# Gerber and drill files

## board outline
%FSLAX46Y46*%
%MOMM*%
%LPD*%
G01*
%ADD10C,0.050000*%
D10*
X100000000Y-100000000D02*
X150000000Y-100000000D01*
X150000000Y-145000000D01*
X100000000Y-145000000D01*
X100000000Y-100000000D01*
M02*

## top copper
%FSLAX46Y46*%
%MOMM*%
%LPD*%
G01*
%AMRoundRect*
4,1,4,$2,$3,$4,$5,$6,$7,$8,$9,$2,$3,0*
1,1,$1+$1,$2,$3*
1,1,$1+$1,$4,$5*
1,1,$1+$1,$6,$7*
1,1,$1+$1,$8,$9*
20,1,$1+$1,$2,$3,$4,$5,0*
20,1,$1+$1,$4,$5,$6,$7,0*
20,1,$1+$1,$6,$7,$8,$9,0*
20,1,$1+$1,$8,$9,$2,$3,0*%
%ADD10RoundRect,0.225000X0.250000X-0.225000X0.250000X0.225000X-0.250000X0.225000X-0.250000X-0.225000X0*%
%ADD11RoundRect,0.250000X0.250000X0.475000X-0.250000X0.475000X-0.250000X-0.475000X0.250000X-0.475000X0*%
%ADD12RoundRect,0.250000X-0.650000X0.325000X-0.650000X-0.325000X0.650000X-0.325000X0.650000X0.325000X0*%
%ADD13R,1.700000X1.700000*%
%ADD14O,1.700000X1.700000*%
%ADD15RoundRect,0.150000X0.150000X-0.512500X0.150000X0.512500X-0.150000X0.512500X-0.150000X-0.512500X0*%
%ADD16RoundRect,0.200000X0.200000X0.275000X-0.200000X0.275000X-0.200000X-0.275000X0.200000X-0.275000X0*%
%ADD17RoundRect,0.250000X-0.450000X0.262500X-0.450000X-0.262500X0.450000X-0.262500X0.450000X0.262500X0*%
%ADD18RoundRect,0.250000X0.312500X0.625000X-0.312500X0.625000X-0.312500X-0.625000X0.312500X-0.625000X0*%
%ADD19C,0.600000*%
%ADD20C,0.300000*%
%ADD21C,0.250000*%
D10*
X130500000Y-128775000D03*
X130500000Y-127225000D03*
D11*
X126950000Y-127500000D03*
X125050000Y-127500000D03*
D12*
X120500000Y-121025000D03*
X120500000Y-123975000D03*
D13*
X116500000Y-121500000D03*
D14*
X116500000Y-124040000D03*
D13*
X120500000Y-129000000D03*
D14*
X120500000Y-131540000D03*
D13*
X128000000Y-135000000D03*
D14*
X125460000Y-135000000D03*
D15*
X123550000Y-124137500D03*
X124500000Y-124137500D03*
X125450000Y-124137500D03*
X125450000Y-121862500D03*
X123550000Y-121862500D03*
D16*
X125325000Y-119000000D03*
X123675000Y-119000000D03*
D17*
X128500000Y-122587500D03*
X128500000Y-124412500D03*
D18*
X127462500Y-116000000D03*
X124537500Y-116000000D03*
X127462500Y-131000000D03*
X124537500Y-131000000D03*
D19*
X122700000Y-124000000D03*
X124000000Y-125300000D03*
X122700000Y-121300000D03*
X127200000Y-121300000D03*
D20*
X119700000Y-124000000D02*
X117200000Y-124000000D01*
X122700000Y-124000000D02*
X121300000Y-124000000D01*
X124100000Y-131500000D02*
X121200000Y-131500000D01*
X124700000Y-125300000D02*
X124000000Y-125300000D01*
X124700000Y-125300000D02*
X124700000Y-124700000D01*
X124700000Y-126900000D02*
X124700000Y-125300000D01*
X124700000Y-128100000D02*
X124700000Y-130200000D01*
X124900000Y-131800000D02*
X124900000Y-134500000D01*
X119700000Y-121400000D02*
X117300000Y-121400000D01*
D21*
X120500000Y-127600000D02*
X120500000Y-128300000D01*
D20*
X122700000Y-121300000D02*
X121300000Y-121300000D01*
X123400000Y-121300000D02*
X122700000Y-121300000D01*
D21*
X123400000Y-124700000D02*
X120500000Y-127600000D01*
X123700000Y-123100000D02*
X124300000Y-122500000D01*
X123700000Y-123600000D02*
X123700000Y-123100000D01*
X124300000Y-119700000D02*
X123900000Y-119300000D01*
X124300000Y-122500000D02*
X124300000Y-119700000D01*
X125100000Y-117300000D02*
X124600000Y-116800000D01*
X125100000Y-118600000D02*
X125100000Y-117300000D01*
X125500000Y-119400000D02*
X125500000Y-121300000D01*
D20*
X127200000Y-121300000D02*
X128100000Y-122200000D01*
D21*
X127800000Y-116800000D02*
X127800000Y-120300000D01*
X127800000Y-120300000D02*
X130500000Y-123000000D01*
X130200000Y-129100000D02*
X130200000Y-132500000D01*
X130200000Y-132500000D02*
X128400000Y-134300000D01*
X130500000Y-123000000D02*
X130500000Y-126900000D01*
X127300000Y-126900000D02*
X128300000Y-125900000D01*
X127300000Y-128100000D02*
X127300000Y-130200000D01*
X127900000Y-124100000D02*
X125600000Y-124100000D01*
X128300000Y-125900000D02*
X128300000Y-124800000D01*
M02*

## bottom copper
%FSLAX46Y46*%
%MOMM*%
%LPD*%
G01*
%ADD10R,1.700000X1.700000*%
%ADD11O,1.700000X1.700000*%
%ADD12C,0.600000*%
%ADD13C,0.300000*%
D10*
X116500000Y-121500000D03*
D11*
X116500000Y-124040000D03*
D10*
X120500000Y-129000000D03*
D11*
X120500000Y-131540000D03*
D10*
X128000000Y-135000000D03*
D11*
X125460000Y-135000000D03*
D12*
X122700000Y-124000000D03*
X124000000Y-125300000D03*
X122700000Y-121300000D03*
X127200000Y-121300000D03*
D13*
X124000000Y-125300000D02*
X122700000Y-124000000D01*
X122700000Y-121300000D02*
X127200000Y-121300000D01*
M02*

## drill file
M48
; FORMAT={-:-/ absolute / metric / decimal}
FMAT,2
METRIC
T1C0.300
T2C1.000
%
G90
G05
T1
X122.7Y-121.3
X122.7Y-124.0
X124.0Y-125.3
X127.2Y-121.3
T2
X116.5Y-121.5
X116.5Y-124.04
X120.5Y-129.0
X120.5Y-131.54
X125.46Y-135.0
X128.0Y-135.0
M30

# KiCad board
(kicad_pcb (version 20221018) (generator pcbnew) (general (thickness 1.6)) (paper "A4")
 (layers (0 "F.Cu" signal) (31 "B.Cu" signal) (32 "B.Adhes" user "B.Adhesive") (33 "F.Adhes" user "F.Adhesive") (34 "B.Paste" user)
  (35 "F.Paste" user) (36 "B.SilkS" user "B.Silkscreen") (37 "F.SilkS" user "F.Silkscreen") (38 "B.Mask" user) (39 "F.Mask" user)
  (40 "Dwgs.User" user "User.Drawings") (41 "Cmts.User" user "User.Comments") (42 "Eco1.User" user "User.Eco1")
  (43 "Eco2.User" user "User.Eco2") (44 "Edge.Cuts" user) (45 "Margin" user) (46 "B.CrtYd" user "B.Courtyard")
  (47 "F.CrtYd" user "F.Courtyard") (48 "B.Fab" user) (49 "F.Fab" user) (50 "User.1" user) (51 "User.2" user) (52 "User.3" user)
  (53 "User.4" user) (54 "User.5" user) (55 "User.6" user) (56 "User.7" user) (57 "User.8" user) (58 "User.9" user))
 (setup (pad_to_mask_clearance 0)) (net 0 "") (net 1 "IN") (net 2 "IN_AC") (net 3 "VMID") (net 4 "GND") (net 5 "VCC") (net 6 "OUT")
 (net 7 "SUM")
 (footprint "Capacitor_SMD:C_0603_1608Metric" (layer "F.Cu") (at 130.5 128 90)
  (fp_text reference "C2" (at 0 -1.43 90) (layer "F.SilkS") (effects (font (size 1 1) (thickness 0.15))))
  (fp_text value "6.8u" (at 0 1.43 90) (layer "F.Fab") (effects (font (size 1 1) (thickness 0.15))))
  (pad "1" smd roundrect (at -0.775 0 90) (size 0.9 0.95) (layers "F.Cu" "F.Paste" "F.Mask") (roundrect_rratio 0.25) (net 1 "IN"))
  (pad "2" smd roundrect (at 0.775 0 90) (size 0.9 0.95) (layers "F.Cu" "F.Paste" "F.Mask") (roundrect_rratio 0.25) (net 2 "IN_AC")))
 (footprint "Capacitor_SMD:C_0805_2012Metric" (layer "F.Cu") (at 126 127.5 180)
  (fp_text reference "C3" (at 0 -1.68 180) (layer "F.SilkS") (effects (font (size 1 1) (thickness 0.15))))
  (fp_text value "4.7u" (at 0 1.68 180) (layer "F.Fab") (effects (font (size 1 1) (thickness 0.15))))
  (pad "1" smd roundrect (at -0.95 0 180) (size 1 1.45) (layers "F.Cu" "F.Paste" "F.Mask") (roundrect_rratio 0.25) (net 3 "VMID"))
  (pad "2" smd roundrect (at 0.95 0 180) (size 1 1.45) (layers "F.Cu" "F.Paste" "F.Mask") (roundrect_rratio 0.25) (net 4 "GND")))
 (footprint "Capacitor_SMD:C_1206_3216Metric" (layer "F.Cu") (at 120.5 122.5 -90)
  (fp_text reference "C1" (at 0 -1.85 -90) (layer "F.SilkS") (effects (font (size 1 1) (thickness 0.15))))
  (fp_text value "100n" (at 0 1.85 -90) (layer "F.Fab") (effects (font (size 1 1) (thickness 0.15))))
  (pad "1" smd roundrect (at -1.475 0 270) (size 1.15 1.8) (layers "F.Cu" "F.Paste" "F.Mask") (roundrect_rratio 0.217391) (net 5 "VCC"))
  (pad "2" smd roundrect (at 1.475 0 270) (size 1.15 1.8) (layers "F.Cu" "F.Paste" "F.Mask") (roundrect_rratio 0.217391) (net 4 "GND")))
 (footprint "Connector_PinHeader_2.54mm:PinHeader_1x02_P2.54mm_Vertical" (layer "F.Cu") (at 116.5 121.5)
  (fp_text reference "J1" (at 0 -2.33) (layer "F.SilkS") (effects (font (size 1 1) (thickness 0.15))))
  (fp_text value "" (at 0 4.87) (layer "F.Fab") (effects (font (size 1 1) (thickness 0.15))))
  (pad "1" thru_hole rect (at 0 0) (size 1.7 1.7) (drill 1) (layers "*.Cu" "*.Mask") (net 5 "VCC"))
  (pad "2" thru_hole oval (at 0 2.54) (size 1.7 1.7) (drill 1) (layers "*.Cu" "*.Mask") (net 4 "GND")))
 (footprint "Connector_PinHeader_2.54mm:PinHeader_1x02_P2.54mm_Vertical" (layer "F.Cu") (at 120.5 129)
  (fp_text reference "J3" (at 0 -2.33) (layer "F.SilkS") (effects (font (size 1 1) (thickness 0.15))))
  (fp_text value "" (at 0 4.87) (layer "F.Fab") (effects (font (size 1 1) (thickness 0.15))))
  (pad "1" thru_hole rect (at 0 0) (size 1.7 1.7) (drill 1) (layers "*.Cu" "*.Mask") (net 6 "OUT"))
  (pad "2" thru_hole oval (at 0 2.54) (size 1.7 1.7) (drill 1) (layers "*.Cu" "*.Mask") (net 4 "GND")))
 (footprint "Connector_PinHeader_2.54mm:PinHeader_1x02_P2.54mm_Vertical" (layer "F.Cu") (at 128 135 -90)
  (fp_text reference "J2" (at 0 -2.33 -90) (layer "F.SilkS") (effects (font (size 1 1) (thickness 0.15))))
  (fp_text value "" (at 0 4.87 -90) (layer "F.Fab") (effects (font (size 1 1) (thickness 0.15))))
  (pad "1" thru_hole rect (at 0 0 270) (size 1.7 1.7) (drill 1) (layers "*.Cu" "*.Mask") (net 1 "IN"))
  (pad "2" thru_hole oval (at 0 2.54 270) (size 1.7 1.7) (drill 1) (layers "*.Cu" "*.Mask") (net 4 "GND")))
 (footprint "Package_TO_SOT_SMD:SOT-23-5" (layer "F.Cu") (at 124.5 123 90)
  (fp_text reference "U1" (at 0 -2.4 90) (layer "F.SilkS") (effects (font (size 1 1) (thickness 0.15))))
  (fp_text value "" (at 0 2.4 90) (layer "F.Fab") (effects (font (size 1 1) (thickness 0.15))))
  (pad "1" smd roundrect (at -1.1375 -0.95 90) (size 1.325 0.6) (layers "F.Cu" "F.Paste" "F.Mask") (roundrect_rratio 0.25) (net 6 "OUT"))
  (pad "2" smd roundrect (at -1.1375 0 90) (size 1.325 0.6) (layers "F.Cu" "F.Paste" "F.Mask") (roundrect_rratio 0.25) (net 4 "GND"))
  (pad "3" smd roundrect (at -1.1375 0.95 90) (size 1.325 0.6) (layers "F.Cu" "F.Paste" "F.Mask") (roundrect_rratio 0.25) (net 3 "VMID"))
  (pad "4" smd roundrect (at 1.1375 0.95 90) (size 1.325 0.6) (layers "F.Cu" "F.Paste" "F.Mask") (roundrect_rratio 0.25) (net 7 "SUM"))
  (pad "5" smd roundrect (at 1.1375 -0.95 90) (size 1.325 0.6) (layers "F.Cu" "F.Paste" "F.Mask") (roundrect_rratio 0.25) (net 5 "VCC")))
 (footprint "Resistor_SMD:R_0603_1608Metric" (layer "F.Cu") (at 124.5 119 180)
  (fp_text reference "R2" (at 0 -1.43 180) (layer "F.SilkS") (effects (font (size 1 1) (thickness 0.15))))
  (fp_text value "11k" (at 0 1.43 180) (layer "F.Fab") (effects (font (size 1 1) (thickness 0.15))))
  (pad "1" smd roundrect (at -0.825 0 180) (size 0.8 0.95) (layers "F.Cu" "F.Paste" "F.Mask") (roundrect_rratio 0.25) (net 7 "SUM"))
  (pad "2" smd roundrect (at 0.825 0 180) (size 0.8 0.95) (layers "F.Cu" "F.Paste" "F.Mask") (roundrect_rratio 0.25) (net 6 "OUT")))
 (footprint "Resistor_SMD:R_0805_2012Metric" (layer "F.Cu") (at 128.5 123.5 -90)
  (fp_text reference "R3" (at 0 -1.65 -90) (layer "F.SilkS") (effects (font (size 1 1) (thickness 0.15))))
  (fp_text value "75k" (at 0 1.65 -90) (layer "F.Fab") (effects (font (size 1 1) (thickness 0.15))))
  (pad "1" smd roundrect (at -0.9125 0 270) (size 1.025 1.4) (layers "F.Cu" "F.Paste" "F.Mask") (roundrect_rratio 0.243902) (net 5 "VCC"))
  (pad "2" smd roundrect (at 0.9125 0 270) (size 1.025 1.4) (layers "F.Cu" "F.Paste" "F.Mask") (roundrect_rratio 0.243902) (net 3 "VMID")))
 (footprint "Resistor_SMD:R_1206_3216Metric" (layer "F.Cu") (at 126 116 180)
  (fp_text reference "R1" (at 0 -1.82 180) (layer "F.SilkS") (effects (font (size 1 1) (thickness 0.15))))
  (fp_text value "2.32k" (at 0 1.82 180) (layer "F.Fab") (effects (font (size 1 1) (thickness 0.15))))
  (pad "1" smd roundrect (at -1.4625 0 180) (size 1.125 1.75) (layers "F.Cu" "F.Paste" "F.Mask") (roundrect_rratio 0.222222) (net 2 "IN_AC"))
  (pad "2" smd roundrect (at 1.4625 0 180) (size 1.125 1.75) (layers "F.Cu" "F.Paste" "F.Mask") (roundrect_rratio 0.222222) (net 7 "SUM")))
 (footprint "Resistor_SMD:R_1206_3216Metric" (layer "F.Cu") (at 126 131 180)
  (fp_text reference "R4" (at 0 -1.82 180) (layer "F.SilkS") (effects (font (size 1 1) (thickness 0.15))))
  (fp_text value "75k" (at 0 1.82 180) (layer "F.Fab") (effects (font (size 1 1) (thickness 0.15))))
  (pad "1" smd roundrect (at -1.4625 0 180) (size 1.125 1.75) (layers "F.Cu" "F.Paste" "F.Mask") (roundrect_rratio 0.222222) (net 3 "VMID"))
  (pad "2" smd roundrect (at 1.4625 0 180) (size 1.125 1.75) (layers "F.Cu" "F.Paste" "F.Mask") (roundrect_rratio 0.222222) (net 4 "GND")))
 (gr_rect (start 100 100) (end 150 145) (stroke (width 0.05) (type default)) (fill none) (layer "Edge.Cuts"))
 (segment (start 119.7 124) (end 117.2 124) (width 0.3) (layer "F.Cu") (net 4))
 (segment (start 122.7 124) (end 121.3 124) (width 0.3) (layer "F.Cu") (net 4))
 (segment (start 124.1 131.5) (end 121.2 131.5) (width 0.3) (layer "F.Cu") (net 4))
 (segment (start 124.7 125.3) (end 124 125.3) (width 0.3) (layer "F.Cu") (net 4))
 (segment (start 124.7 125.3) (end 124.7 124.7) (width 0.3) (layer "F.Cu") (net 4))
 (segment (start 124.7 126.9) (end 124.7 125.3) (width 0.3) (layer "F.Cu") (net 4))
 (segment (start 124.7 128.1) (end 124.7 130.2) (width 0.3) (layer "F.Cu") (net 4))
 (segment (start 124.9 131.8) (end 124.9 134.5) (width 0.3) (layer "F.Cu") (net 4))
 (via (at 122.7 124) (size 0.6) (drill 0.3) (layers "F.Cu" "B.Cu") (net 4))
 (via (at 124 125.3) (size 0.6) (drill 0.3) (layers "F.Cu" "B.Cu") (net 4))
 (segment (start 119.7 121.4) (end 117.3 121.4) (width 0.3) (layer "F.Cu") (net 5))
 (segment (start 120.5 127.6) (end 120.5 128.3) (width 0.25) (layer "F.Cu") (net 6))
 (segment (start 122.7 121.3) (end 121.3 121.3) (width 0.3) (layer "F.Cu") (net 5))
 (segment (start 123.4 121.3) (end 122.7 121.3) (width 0.3) (layer "F.Cu") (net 5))
 (segment (start 123.4 124.7) (end 120.5 127.6) (width 0.25) (layer "F.Cu") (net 6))
 (segment (start 123.7 123.1) (end 124.3 122.5) (width 0.25) (layer "F.Cu") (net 6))
 (segment (start 123.7 123.6) (end 123.7 123.1) (width 0.25) (layer "F.Cu") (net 6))
 (segment (start 124 125.3) (end 122.7 124) (width 0.3) (layer "B.Cu") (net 4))
 (segment (start 124.3 119.7) (end 123.9 119.3) (width 0.25) (layer "F.Cu") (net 6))
 (segment (start 124.3 122.5) (end 124.3 119.7) (width 0.25) (layer "F.Cu") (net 6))
 (segment (start 125.1 117.3) (end 124.6 116.8) (width 0.25) (layer "F.Cu") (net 7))
 (segment (start 125.1 118.6) (end 125.1 117.3) (width 0.25) (layer "F.Cu") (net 7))
 (segment (start 125.5 119.4) (end 125.5 121.3) (width 0.25) (layer "F.Cu") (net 7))
 (segment (start 127.2 121.3) (end 128.1 122.2) (width 0.3) (layer "F.Cu") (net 5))
 (segment (start 127.8 116.8) (end 127.8 120.3) (width 0.25) (layer "F.Cu") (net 2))
 (segment (start 127.8 120.3) (end 130.5 123) (width 0.25) (layer "F.Cu") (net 2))
 (segment (start 130.2 129.1) (end 130.2 132.5) (width 0.25) (layer "F.Cu") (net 1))
 (segment (start 130.2 132.5) (end 128.4 134.3) (width 0.25) (layer "F.Cu") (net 1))
 (segment (start 130.5 123) (end 130.5 126.9) (width 0.25) (layer "F.Cu") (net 2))
 (via (at 122.7 121.3) (size 0.6) (drill 0.3) (layers "F.Cu" "B.Cu") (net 5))
 (via (at 127.2 121.3) (size 0.6) (drill 0.3) (layers "F.Cu" "B.Cu") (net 5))
 (segment (start 122.7 121.3) (end 127.2 121.3) (width 0.3) (layer "B.Cu") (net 5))
 (segment (start 127.3 126.9) (end 128.3 125.9) (width 0.25) (layer "F.Cu") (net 3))
 (segment (start 127.3 128.1) (end 127.3 130.2) (width 0.25) (layer "F.Cu") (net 3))
 (segment (start 127.9 124.1) (end 125.6 124.1) (width 0.25) (layer "F.Cu") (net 3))
 (segment (start 128.3 125.9) (end 128.3 124.8) (width 0.25) (layer "F.Cu") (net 3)))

